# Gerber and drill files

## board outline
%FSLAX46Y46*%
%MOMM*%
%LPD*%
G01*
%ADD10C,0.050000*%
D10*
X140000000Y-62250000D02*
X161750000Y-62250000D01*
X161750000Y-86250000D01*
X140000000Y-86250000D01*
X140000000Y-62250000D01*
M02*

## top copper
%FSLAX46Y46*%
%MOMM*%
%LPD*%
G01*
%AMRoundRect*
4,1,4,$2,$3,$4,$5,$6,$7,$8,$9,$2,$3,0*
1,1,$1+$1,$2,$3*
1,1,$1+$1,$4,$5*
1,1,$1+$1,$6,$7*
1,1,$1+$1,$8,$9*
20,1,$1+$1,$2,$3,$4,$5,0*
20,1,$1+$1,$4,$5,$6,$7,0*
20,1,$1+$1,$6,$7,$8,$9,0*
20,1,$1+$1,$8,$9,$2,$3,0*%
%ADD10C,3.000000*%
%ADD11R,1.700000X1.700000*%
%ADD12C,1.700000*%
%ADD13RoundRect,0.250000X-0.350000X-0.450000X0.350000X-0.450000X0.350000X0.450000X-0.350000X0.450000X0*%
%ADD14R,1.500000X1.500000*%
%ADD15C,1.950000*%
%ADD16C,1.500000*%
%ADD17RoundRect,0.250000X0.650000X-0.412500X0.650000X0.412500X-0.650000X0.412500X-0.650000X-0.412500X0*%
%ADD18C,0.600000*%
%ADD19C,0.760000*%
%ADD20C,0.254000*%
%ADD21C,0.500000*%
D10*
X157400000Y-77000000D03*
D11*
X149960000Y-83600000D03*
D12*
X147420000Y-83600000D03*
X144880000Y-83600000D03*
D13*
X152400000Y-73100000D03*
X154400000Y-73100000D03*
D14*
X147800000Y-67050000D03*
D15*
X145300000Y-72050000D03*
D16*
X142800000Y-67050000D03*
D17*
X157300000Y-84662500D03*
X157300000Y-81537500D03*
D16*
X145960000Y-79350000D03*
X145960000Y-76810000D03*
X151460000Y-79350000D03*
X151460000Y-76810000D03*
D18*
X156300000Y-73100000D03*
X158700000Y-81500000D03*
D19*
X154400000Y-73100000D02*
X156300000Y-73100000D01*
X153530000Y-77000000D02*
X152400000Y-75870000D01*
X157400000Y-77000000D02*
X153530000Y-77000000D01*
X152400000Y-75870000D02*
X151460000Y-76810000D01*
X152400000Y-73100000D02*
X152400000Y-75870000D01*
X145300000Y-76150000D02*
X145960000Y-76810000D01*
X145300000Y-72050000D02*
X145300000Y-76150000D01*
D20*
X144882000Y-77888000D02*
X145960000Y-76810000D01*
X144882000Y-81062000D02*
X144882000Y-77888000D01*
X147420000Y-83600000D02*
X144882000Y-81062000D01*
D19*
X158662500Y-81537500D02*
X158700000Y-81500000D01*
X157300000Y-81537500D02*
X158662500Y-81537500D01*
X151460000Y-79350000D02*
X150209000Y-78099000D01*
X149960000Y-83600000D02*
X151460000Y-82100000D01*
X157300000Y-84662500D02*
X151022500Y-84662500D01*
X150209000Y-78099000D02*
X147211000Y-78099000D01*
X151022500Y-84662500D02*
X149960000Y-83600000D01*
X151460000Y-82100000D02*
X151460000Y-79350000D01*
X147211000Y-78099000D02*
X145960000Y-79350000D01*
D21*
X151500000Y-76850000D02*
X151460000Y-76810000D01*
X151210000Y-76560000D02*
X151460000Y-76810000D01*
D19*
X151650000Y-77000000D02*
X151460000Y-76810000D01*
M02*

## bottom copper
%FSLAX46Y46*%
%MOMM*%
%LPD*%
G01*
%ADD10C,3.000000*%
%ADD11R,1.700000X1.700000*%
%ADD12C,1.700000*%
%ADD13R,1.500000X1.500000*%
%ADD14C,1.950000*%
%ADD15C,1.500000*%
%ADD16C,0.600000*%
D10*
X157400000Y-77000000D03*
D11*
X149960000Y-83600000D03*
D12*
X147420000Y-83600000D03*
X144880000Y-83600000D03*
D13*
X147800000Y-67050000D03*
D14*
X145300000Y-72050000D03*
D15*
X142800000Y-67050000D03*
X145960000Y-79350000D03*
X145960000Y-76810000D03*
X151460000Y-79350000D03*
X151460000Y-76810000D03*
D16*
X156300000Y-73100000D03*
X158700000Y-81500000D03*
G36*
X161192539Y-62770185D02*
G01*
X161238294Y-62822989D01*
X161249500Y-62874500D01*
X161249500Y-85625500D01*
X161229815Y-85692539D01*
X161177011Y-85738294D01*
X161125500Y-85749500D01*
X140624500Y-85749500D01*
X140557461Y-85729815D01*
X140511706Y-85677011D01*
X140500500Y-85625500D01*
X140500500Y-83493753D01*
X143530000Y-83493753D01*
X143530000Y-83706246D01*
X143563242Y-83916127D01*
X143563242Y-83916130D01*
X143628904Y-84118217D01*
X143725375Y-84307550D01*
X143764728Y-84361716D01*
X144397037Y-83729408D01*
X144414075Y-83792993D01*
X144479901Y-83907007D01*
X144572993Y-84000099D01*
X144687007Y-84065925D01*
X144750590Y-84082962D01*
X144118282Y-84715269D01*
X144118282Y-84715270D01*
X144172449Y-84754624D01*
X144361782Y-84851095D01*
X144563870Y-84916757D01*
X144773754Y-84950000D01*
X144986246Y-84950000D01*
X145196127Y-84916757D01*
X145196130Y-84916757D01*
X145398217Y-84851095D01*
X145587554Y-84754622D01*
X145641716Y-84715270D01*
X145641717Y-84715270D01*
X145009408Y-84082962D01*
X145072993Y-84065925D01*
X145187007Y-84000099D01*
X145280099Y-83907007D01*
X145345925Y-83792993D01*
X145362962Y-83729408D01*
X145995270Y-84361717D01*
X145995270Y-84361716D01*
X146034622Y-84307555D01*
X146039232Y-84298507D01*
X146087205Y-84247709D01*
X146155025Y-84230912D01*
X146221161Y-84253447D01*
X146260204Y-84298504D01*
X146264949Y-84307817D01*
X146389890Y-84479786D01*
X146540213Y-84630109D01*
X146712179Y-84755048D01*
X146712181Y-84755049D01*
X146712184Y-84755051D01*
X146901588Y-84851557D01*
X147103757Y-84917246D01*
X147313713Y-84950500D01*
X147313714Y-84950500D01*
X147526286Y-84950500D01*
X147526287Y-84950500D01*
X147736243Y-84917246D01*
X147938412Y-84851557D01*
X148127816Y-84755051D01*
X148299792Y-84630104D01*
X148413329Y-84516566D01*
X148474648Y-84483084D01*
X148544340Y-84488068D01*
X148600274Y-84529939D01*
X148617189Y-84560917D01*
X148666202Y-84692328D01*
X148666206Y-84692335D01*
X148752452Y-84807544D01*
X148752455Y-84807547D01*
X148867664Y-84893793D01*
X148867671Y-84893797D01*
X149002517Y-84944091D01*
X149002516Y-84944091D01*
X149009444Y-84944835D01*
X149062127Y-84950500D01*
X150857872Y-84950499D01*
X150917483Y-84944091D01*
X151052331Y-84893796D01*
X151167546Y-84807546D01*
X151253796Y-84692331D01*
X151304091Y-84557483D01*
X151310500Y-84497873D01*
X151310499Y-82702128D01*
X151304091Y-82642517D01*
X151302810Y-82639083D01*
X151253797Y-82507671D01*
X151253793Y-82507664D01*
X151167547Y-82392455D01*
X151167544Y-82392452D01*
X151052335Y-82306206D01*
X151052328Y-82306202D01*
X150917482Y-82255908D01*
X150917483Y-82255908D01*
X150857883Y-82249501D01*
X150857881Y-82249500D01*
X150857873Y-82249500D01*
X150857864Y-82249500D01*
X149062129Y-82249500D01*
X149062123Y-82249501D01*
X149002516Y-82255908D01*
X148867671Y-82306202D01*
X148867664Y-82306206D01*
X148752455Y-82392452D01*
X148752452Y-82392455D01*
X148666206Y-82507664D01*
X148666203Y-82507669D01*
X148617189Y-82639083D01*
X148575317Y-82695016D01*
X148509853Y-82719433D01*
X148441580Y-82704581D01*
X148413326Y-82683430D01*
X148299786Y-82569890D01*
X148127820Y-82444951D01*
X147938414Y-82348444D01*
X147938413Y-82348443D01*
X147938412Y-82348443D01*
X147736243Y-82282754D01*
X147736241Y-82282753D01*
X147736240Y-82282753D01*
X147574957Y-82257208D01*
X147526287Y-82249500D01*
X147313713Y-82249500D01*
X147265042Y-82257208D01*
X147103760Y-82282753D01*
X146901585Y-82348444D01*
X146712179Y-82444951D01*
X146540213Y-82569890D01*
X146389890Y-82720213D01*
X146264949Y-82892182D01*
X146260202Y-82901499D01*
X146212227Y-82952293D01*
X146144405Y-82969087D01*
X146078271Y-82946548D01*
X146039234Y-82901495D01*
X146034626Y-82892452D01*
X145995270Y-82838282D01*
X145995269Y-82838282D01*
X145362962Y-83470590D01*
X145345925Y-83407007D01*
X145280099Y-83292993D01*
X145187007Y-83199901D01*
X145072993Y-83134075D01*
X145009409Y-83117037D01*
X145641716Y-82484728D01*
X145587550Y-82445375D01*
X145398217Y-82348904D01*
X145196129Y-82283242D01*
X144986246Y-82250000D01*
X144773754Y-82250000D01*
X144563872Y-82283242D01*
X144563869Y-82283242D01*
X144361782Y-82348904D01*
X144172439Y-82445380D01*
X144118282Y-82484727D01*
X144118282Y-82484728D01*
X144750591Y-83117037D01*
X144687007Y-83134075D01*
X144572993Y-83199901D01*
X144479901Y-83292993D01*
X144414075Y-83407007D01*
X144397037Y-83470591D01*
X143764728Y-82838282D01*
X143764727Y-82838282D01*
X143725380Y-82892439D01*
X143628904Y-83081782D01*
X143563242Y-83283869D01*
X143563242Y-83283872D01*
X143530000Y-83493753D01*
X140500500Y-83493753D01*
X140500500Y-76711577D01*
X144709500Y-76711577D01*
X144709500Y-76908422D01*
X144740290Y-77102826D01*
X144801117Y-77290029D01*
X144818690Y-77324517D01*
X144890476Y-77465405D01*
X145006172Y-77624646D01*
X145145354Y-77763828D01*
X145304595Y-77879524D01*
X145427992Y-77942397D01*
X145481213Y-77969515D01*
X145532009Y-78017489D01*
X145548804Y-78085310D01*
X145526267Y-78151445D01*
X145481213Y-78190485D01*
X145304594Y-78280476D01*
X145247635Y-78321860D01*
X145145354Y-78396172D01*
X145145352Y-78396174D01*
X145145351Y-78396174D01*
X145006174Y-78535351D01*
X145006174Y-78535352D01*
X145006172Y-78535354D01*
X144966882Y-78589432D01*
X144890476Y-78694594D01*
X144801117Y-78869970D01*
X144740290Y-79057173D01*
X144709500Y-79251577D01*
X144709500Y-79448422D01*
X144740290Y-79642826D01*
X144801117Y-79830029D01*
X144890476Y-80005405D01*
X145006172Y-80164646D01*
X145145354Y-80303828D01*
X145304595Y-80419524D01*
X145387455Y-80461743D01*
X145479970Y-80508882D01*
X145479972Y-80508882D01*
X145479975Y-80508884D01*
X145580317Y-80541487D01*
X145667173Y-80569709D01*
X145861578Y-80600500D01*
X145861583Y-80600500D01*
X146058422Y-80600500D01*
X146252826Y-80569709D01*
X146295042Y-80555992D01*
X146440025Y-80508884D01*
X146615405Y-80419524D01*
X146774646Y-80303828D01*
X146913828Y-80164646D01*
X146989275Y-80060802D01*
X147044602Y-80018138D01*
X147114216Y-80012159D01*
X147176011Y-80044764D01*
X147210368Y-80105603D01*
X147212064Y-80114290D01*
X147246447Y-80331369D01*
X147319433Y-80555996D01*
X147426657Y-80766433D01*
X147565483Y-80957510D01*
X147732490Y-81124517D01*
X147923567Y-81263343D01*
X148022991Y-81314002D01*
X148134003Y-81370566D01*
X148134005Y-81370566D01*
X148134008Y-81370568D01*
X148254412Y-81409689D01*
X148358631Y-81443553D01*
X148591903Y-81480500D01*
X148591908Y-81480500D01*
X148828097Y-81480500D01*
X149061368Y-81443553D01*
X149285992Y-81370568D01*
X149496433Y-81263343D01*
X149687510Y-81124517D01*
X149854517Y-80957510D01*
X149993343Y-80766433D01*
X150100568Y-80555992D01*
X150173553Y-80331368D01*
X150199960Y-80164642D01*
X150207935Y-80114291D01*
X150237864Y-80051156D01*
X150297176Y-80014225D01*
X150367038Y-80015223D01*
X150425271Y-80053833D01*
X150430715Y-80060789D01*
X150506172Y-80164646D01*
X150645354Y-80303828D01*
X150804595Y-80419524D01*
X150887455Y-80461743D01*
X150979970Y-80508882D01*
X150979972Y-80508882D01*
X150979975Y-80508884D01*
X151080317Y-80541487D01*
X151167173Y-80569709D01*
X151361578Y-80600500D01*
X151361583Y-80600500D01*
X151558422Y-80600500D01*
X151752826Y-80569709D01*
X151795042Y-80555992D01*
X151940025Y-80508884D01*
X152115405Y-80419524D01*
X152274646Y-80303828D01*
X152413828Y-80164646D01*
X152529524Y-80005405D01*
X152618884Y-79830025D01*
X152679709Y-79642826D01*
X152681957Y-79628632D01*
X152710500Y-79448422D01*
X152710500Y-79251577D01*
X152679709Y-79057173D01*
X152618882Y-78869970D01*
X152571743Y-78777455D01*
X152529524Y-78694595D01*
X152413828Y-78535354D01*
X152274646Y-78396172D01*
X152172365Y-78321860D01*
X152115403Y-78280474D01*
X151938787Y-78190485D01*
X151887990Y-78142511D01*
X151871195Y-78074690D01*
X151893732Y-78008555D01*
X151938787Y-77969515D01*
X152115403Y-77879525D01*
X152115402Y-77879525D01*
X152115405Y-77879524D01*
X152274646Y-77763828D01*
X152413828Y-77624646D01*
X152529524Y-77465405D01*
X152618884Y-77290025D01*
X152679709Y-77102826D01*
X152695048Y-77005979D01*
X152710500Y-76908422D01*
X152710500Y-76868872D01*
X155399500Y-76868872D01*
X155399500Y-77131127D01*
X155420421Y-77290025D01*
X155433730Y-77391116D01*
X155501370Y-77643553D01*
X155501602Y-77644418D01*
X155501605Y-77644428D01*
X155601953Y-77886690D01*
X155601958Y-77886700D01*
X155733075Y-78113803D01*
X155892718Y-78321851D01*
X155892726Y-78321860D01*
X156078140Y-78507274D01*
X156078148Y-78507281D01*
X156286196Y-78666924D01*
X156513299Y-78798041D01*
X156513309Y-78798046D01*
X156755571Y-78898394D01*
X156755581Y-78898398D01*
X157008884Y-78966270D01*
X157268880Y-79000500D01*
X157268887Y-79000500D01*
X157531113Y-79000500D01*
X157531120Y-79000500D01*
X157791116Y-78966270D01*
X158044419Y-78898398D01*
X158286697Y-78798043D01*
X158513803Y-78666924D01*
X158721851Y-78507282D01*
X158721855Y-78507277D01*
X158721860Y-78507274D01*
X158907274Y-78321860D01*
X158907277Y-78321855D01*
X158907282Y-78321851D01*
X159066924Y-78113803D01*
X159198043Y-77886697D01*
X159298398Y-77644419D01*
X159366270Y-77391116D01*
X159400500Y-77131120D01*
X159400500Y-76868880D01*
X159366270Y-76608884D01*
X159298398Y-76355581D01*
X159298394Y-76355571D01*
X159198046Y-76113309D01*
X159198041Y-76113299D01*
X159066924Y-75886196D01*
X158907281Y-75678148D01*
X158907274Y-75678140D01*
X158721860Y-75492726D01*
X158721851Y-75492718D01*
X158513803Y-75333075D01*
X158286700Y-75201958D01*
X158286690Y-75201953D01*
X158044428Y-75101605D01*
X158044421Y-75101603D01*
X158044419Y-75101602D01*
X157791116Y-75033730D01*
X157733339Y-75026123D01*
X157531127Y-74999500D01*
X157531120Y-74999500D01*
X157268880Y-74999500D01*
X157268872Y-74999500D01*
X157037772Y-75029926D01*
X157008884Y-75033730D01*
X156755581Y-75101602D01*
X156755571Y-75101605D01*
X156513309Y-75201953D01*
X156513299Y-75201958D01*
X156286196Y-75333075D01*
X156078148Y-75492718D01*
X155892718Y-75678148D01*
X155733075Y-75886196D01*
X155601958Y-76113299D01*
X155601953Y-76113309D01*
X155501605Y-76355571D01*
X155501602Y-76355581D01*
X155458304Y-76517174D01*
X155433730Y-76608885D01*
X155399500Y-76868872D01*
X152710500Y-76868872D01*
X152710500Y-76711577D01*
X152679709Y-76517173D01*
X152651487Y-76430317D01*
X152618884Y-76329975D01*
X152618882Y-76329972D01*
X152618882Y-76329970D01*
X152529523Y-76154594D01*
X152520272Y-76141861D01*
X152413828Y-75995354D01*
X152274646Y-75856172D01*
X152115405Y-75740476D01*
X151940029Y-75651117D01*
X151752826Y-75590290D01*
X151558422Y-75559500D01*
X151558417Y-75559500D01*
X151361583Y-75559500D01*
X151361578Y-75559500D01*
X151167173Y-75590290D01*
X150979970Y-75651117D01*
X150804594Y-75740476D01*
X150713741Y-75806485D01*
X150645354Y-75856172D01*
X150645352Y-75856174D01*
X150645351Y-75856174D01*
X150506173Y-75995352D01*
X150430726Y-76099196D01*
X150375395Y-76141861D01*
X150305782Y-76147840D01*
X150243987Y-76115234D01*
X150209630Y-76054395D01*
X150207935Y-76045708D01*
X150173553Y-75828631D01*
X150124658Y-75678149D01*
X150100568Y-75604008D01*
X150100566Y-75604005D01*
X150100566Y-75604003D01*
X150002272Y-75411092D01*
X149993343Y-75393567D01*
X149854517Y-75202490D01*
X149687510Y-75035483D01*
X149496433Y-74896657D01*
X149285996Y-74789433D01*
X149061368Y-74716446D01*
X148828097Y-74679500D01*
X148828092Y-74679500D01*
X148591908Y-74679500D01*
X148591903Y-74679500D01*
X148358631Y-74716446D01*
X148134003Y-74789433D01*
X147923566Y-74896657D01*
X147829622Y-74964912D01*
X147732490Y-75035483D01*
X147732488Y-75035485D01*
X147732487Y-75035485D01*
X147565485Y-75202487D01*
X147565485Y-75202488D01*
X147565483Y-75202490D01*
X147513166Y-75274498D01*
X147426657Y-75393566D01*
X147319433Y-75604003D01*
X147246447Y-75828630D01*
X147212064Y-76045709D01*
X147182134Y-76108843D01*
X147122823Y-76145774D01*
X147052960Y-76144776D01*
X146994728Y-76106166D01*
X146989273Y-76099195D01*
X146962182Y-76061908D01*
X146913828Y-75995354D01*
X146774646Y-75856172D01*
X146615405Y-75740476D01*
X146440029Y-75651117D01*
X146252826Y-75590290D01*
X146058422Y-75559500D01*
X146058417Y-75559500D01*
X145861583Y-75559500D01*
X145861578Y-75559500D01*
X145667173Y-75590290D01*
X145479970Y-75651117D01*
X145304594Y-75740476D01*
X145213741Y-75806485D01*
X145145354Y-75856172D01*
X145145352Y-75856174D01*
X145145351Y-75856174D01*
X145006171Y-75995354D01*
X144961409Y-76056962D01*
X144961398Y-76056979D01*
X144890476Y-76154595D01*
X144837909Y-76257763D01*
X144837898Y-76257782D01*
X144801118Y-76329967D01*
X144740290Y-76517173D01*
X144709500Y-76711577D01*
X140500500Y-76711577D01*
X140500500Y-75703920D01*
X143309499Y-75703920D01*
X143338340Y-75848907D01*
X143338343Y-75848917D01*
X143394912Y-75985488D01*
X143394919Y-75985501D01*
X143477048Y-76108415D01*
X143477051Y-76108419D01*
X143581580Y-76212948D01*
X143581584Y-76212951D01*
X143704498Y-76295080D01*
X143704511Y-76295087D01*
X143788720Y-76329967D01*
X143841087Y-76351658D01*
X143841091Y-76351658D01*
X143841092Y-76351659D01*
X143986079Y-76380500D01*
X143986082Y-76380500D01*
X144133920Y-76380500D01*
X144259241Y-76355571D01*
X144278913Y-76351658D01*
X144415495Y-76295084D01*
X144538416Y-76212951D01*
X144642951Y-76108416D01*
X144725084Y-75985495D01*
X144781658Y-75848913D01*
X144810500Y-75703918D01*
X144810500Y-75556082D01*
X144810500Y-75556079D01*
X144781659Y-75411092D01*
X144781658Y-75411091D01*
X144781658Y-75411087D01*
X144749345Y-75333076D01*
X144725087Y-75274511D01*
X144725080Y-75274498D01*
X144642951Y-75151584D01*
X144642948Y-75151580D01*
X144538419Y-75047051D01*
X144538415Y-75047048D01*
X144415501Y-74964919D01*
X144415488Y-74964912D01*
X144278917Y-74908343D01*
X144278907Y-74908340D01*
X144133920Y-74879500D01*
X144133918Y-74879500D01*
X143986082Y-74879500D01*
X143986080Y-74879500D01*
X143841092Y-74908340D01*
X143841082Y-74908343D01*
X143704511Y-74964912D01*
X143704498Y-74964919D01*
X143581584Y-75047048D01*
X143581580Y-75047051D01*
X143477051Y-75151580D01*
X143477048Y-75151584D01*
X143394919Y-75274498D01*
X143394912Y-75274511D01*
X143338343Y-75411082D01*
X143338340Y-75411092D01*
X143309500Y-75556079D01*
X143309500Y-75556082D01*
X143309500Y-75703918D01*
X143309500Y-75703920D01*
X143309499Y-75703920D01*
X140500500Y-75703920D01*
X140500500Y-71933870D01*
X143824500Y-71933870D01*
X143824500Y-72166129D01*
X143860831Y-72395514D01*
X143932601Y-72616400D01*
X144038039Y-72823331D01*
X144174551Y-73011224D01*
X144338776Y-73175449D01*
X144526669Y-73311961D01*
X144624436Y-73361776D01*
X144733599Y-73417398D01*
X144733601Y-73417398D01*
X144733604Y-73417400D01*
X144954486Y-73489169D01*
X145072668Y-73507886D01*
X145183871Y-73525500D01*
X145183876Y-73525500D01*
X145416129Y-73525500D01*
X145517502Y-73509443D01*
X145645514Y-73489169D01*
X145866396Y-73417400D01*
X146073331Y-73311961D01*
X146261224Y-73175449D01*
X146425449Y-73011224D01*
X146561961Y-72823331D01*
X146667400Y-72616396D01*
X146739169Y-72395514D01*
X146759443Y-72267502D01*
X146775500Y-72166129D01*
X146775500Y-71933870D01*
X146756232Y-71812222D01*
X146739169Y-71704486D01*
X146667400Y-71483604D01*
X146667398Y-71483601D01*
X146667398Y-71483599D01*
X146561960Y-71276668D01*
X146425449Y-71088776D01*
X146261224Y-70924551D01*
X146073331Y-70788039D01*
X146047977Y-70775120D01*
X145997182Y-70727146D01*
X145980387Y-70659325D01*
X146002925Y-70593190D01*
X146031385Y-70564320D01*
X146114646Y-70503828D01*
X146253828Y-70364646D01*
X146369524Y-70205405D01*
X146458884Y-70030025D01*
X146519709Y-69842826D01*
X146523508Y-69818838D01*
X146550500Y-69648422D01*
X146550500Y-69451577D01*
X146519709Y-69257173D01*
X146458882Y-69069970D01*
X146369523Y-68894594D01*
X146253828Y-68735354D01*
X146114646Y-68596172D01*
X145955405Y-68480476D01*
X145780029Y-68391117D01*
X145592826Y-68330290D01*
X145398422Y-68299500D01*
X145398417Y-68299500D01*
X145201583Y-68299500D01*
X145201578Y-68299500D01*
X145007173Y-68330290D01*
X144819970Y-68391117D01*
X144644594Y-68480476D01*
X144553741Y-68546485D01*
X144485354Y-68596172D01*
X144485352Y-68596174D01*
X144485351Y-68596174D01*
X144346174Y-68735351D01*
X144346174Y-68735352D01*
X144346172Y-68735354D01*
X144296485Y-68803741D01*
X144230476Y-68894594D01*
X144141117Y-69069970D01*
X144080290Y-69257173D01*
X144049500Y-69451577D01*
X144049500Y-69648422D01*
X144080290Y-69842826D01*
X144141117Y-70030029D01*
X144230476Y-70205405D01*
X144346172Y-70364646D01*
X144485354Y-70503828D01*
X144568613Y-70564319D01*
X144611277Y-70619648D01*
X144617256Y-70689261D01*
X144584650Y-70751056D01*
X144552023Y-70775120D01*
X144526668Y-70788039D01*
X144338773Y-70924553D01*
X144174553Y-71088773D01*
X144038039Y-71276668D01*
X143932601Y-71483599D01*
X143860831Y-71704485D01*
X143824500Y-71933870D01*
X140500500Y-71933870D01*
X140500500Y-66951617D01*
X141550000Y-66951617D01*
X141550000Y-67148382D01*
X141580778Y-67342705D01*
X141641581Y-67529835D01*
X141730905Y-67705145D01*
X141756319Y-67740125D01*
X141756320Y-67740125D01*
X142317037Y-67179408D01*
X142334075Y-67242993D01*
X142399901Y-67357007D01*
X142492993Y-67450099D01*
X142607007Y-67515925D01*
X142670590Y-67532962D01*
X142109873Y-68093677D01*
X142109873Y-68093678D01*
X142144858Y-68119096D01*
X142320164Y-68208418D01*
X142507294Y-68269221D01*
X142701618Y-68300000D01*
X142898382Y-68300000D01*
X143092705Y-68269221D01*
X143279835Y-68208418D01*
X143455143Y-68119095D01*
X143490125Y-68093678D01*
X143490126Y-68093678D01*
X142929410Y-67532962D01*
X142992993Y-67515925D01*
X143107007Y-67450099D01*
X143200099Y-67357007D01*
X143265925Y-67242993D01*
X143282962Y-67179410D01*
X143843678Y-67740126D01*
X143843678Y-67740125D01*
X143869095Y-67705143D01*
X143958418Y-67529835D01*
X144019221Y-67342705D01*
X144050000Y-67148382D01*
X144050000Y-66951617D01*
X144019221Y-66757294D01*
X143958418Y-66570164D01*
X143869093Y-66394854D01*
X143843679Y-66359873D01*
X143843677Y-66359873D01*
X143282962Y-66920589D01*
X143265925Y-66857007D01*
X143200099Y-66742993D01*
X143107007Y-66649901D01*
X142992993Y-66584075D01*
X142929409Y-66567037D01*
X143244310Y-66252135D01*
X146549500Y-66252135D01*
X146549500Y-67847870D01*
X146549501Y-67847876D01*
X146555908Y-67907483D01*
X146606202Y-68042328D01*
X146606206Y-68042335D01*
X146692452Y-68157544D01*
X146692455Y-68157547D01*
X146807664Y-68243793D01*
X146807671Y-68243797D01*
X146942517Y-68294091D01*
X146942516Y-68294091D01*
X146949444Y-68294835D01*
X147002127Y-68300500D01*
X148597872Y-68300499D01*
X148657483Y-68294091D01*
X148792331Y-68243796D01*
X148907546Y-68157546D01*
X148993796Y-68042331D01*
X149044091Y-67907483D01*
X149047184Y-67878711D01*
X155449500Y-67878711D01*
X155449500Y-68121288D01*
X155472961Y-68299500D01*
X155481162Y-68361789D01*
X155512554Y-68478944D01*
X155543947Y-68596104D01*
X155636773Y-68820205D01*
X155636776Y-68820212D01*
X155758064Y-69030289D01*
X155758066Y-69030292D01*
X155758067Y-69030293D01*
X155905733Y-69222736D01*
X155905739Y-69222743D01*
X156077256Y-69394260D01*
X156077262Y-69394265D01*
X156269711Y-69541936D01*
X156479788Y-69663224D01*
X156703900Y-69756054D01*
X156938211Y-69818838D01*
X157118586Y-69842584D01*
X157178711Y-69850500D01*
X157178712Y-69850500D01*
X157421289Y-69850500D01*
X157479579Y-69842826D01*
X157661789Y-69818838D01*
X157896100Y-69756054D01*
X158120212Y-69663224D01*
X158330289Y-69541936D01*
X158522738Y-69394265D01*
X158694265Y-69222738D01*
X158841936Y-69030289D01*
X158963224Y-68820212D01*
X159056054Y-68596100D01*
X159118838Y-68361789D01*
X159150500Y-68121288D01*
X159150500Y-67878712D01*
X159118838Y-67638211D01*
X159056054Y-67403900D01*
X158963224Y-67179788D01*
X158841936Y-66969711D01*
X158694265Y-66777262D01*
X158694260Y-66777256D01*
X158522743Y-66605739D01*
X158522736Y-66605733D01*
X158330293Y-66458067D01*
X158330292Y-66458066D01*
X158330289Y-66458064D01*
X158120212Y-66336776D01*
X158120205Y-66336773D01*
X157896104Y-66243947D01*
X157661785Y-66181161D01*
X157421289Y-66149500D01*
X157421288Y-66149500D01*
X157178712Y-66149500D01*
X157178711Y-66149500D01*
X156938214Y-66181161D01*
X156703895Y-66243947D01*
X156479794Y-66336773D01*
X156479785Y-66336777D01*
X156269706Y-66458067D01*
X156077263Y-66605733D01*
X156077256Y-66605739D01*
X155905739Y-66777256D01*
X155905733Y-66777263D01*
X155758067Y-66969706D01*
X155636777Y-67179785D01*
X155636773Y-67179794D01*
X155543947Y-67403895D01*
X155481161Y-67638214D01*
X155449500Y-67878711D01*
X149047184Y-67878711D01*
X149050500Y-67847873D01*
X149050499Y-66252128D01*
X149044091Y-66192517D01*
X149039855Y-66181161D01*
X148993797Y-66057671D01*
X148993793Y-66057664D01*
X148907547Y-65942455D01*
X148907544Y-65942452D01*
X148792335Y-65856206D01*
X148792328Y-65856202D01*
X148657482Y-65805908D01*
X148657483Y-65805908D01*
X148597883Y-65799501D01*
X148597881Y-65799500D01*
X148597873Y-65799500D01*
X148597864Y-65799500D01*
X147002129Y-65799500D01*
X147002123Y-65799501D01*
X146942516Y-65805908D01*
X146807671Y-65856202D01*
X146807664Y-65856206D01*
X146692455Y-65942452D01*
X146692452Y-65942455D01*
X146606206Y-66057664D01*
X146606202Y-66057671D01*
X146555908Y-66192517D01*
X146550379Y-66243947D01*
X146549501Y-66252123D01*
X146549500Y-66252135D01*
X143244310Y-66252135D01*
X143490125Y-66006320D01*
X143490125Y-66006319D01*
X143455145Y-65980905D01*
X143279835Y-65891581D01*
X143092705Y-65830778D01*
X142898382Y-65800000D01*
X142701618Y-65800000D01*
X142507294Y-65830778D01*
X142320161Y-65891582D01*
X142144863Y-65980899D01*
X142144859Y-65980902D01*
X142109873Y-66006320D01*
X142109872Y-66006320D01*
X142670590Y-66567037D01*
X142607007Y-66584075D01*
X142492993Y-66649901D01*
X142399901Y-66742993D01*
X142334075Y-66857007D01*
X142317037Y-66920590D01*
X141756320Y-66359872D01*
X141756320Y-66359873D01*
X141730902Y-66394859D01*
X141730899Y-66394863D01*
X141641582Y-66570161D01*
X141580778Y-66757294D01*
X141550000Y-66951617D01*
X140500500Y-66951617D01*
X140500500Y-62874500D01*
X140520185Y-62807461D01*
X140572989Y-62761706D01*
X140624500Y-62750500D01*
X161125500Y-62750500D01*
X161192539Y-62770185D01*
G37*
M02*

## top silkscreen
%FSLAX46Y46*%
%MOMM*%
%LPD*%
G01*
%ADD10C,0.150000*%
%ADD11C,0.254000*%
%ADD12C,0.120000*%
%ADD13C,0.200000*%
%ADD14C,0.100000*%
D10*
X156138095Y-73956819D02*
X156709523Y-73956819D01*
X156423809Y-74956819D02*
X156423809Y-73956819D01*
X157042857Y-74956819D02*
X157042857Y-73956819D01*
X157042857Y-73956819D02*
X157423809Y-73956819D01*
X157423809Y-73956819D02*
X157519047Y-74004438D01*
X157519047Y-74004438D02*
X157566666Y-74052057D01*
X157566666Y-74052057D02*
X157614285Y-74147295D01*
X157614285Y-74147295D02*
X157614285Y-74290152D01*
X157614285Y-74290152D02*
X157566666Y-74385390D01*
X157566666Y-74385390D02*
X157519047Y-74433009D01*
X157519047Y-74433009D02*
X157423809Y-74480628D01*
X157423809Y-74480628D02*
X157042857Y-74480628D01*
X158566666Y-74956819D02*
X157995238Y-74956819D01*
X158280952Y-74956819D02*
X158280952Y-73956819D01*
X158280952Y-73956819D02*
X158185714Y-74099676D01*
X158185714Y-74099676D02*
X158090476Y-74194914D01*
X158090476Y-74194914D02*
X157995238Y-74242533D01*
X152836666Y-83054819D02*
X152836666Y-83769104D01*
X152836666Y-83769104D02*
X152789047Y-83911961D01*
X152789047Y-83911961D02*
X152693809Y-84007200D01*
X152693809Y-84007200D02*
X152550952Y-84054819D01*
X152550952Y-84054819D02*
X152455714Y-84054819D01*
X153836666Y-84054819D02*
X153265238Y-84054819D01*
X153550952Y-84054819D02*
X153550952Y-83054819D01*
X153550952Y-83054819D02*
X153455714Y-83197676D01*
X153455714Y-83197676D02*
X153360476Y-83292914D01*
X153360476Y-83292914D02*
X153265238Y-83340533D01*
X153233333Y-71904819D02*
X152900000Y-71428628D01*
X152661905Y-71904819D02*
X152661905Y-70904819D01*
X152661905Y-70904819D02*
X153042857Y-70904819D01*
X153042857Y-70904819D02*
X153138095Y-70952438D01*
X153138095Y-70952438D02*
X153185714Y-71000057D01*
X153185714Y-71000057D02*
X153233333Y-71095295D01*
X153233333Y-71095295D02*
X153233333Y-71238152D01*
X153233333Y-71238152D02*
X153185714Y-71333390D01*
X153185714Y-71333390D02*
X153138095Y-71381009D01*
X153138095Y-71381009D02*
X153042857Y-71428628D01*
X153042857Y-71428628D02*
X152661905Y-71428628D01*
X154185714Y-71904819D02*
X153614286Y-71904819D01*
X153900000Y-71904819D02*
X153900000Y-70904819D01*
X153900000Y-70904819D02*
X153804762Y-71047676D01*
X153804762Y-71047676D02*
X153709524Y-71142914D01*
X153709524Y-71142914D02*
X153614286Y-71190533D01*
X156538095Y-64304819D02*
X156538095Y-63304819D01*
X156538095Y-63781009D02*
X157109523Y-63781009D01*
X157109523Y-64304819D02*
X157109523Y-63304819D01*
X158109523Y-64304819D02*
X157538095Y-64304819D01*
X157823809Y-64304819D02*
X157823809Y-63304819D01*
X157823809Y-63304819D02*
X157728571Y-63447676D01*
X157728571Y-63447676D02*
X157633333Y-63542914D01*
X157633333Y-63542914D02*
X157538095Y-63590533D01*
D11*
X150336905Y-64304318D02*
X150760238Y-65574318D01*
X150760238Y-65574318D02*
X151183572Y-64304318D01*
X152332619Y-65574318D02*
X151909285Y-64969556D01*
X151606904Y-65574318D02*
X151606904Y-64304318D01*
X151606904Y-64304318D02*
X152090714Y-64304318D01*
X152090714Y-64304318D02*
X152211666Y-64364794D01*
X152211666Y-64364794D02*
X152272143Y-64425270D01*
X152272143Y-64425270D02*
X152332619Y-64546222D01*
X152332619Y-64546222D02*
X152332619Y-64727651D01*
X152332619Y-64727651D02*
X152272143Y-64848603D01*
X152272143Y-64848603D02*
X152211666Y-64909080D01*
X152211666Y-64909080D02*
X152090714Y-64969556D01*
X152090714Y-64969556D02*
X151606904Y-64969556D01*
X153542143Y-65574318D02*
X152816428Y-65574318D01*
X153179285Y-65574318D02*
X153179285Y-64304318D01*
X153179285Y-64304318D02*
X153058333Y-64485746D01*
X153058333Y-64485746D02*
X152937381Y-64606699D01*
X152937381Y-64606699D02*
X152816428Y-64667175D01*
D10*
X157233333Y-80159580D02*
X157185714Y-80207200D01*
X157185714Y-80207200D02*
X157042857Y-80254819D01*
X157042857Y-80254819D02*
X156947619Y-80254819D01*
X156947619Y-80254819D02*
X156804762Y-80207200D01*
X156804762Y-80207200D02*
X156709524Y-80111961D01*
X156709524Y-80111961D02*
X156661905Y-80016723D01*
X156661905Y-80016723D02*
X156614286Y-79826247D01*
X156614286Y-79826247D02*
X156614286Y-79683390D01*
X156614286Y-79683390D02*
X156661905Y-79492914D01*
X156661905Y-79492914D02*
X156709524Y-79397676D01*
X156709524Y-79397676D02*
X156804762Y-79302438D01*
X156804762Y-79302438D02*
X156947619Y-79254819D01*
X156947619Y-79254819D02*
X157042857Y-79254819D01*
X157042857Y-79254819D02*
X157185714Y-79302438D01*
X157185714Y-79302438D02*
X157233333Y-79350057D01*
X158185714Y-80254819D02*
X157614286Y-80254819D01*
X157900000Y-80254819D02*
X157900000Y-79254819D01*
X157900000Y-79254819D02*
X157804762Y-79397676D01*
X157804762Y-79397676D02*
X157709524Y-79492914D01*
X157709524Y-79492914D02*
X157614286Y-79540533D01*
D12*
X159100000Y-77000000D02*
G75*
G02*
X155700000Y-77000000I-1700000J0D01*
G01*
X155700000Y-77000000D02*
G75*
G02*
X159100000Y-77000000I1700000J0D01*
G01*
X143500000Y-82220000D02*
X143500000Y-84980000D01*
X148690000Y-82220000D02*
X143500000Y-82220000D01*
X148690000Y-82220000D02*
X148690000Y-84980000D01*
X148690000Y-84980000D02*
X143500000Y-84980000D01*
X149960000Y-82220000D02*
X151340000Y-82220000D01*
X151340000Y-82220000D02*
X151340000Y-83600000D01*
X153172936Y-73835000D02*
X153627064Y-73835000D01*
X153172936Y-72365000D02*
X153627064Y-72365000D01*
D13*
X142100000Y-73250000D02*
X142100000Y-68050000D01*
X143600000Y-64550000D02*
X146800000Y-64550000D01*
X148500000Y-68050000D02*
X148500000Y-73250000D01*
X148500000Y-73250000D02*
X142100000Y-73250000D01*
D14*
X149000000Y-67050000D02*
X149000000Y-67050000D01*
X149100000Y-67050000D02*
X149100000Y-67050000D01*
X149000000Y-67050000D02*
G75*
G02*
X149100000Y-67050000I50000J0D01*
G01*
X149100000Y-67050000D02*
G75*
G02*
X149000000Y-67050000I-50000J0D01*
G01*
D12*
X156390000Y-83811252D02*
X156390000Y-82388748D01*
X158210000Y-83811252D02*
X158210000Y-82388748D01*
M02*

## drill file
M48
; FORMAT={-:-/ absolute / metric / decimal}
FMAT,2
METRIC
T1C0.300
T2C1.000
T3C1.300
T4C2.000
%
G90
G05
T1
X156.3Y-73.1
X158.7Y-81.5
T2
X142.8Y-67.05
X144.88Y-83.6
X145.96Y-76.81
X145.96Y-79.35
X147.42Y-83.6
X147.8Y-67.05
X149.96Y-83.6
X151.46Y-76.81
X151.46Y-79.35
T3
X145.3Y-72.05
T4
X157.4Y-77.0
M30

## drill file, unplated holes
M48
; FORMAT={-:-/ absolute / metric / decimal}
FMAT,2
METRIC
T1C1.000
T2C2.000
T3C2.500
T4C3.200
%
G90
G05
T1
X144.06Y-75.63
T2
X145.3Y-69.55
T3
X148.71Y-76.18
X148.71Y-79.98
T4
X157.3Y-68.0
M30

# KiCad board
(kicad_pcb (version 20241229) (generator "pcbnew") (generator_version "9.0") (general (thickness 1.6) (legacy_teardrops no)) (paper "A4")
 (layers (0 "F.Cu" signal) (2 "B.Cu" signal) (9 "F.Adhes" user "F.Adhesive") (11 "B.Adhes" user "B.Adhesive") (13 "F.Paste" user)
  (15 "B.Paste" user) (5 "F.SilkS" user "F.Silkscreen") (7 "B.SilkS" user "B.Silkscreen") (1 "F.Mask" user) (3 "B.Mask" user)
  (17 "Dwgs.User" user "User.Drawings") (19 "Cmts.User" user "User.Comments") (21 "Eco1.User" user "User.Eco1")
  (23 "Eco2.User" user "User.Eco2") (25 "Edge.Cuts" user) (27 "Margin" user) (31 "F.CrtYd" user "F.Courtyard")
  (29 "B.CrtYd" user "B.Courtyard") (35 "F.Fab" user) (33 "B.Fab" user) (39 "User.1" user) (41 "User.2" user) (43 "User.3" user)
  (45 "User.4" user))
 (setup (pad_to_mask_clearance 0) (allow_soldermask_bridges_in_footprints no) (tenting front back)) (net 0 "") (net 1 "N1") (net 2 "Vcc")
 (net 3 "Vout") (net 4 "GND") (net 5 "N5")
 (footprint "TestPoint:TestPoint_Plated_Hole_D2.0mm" (layer "F.Cu") (at 157.4 77)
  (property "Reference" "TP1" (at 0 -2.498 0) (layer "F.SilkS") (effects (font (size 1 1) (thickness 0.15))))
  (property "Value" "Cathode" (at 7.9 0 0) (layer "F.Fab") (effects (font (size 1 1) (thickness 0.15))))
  (fp_circle (center 0 0) (end 0 -1.7) (stroke (width 0.12) (type solid)) (fill no) (layer "F.SilkS"))
  (pad "1" thru_hole circle (at 0 0) (size 3 3) (drill 2) (layers "*.Cu" "*.Mask") (remove_unused_layers no) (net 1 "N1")))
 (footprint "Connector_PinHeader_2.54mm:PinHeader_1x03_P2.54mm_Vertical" (layer "F.Cu") (at 149.96 83.6 -90)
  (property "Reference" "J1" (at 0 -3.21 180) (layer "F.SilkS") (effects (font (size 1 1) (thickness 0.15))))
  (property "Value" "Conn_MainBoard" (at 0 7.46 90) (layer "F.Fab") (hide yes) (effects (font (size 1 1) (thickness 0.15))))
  (fp_line (start -1.38 6.46) (end 1.38 6.46) (stroke (width 0.12) (type solid)) (layer "F.SilkS"))
  (fp_line (start -1.38 1.27) (end -1.38 6.46) (stroke (width 0.12) (type solid)) (layer "F.SilkS"))
  (fp_line (start -1.38 1.27) (end 1.38 1.27) (stroke (width 0.12) (type solid)) (layer "F.SilkS"))
  (fp_line (start 1.38 1.27) (end 1.38 6.46) (stroke (width 0.12) (type solid)) (layer "F.SilkS"))
  (fp_line (start -1.38 0) (end -1.38 -1.38) (stroke (width 0.12) (type solid)) (layer "F.SilkS"))
  (fp_line (start -1.38 -1.38) (end 0 -1.38) (stroke (width 0.12) (type solid)) (layer "F.SilkS"))
  (pad "1" thru_hole rect (at 0 0 270) (size 1.7 1.7) (drill 1) (layers "*.Cu" "*.Mask") (remove_unused_layers no) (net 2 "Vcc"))
  (pad "2" thru_hole circle (at 0 2.54 270) (size 1.7 1.7) (drill 1) (layers "*.Cu" "*.Mask") (remove_unused_layers no) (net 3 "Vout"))
  (pad "3" thru_hole circle (at 0 5.08 270) (size 1.7 1.7) (drill 1) (layers "*.Cu" "*.Mask") (remove_unused_layers no) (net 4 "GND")))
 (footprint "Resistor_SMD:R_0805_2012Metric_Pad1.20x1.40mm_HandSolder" (layer "F.Cu") (at 153.4 73.1)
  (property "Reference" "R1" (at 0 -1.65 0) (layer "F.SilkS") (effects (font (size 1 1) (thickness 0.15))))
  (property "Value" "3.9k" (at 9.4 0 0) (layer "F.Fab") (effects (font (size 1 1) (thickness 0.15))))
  (fp_line (start -0.227064 -0.735) (end 0.227064 -0.735) (stroke (width 0.12) (type solid)) (layer "F.SilkS"))
  (fp_line (start -0.227064 0.735) (end 0.227064 0.735) (stroke (width 0.12) (type solid)) (layer "F.SilkS"))
  (pad "1" smd roundrect (at -1 0) (size 1.2 1.4) (layers "F.Cu" "F.Mask" "F.Paste") (roundrect_rratio 0.208333) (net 1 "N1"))
  (pad "2" smd roundrect (at 1 0) (size 1.2 1.4) (layers "F.Cu" "F.Mask" "F.Paste") (roundrect_rratio 0.208333) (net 4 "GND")))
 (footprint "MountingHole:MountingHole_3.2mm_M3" (layer "F.Cu") (at 157.3 68)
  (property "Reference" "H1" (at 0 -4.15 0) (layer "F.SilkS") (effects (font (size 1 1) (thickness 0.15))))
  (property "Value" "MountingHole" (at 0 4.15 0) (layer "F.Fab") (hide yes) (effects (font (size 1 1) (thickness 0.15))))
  (pad "" np_thru_hole circle (at 0 0) (size 3.2 3.2) (drill 3.2) (layers "*.Cu" "*.Mask")))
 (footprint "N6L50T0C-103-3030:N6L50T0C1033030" (layer "F.Cu") (at 147.8 67.05 180)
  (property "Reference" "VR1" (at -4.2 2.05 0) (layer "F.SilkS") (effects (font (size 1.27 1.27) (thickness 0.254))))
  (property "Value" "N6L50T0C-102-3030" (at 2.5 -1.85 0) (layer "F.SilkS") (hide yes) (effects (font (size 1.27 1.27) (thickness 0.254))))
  (fp_line (start 5.7 -6.2) (end 5.7 -1) (stroke (width 0.2) (type solid)) (layer "F.SilkS"))
  (fp_line (start 4.2 2.5) (end 1 2.5) (stroke (width 0.2) (type solid)) (layer "F.SilkS"))
  (fp_line (start -0.7 -1) (end -0.7 -6.2) (stroke (width 0.2) (type solid)) (layer "F.SilkS"))
  (fp_line (start -0.7 -6.2) (end 5.7 -6.2) (stroke (width 0.2) (type solid)) (layer "F.SilkS"))
  (fp_line (start -1.2 0) (end -1.2 0) (stroke (width 0.1) (type solid)) (layer "F.SilkS"))
  (fp_line (start -1.3 0) (end -1.3 0) (stroke (width 0.1) (type solid)) (layer "F.SilkS"))
  (fp_arc (start -1.2 0) (mid -1.25 0.05) (end -1.3 0) (stroke (width 0.1) (type solid)) (layer "F.SilkS"))
  (fp_arc (start -1.3 0) (mid -1.25 -0.05) (end -1.2 0) (stroke (width 0.1) (type solid)) (layer "F.SilkS"))
  (pad "" np_thru_hole circle (at 2.5 -2.5 180) (size 2 2) (drill 2) (layers "*.Cu" "*.Mask"))
  (pad "1" thru_hole rect (at 0 0 180) (size 1.5 1.5) (drill 1) (layers "*.Cu" "*.Mask") (remove_unused_layers no) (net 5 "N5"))
  (pad "2" thru_hole circle (at 2.5 -5 180) (size 1.95 1.95) (drill 1.3) (layers "*.Cu" "*.Mask") (remove_unused_layers no) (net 3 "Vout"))
  (pad "3" thru_hole circle (at 5 0 180) (size 1.5 1.5) (drill 1) (layers "*.Cu" "*.Mask") (remove_unused_layers no) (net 4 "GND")))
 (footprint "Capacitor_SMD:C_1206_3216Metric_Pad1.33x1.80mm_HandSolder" (layer "F.Cu") (at 157.3 83.1 90)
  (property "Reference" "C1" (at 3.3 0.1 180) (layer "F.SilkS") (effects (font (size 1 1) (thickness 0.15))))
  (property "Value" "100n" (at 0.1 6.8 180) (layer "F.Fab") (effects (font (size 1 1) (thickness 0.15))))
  (fp_line (start -0.711252 -0.91) (end 0.711252 -0.91) (stroke (width 0.12) (type solid)) (layer "F.SilkS"))
  (fp_line (start -0.711252 0.91) (end 0.711252 0.91) (stroke (width 0.12) (type solid)) (layer "F.SilkS"))
  (pad "1" smd roundrect (at -1.5625 0 90) (size 1.325 1.8) (layers "F.Cu" "F.Mask" "F.Paste") (roundrect_rratio 0.188679) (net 2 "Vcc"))
  (pad "2" smd roundrect (at 1.5625 0 90) (size 1.325 1.8) (layers "F.Cu" "F.Mask" "F.Paste") (roundrect_rratio 0.188679) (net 4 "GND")))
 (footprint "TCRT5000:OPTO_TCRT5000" (layer "B.Cu") (at 148.71 78.08)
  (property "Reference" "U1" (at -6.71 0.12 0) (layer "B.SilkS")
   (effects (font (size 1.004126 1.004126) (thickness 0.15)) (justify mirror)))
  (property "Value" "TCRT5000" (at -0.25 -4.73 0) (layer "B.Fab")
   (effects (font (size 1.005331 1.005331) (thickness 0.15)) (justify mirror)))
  (pad "" np_thru_hole circle (at -4.65 -2.45) (size 1 1) (drill 1) (layers "*.Cu" "*.Mask"))
  (pad "" np_thru_hole circle (at 0 -1.9) (size 2.5 2.5) (drill 2.5) (layers "*.Cu" "*.Mask"))
  (pad "" np_thru_hole circle (at 0 1.9) (size 2.5 2.5) (drill 2.5) (layers "*.Cu" "*.Mask"))
  (pad "1" thru_hole circle (at -2.75 1.27) (size 1.5 1.5) (drill 1) (layers "*.Cu" "*.Mask") (remove_unused_layers no) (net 2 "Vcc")
   (solder_mask_margin 0.102))
  (pad "2" thru_hole circle (at -2.75 -1.27) (size 1.5 1.5) (drill 1) (layers "*.Cu" "*.Mask") (remove_unused_layers no) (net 3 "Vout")
   (solder_mask_margin 0.102))
  (pad "3" thru_hole circle (at 2.75 1.27) (size 1.5 1.5) (drill 1) (layers "*.Cu" "*.Mask") (remove_unused_layers no) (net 2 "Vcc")
   (solder_mask_margin 0.102))
  (pad "4" thru_hole circle (at 2.75 -1.27) (size 1.5 1.5) (drill 1) (layers "*.Cu" "*.Mask") (remove_unused_layers no) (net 1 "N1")
   (solder_mask_margin 0.102)))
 (gr_rect (start 140 62.25) (end 161.75 86.25) (stroke (width 0.05) (type default)) (fill no) (locked yes) (layer "Edge.Cuts"))
 (segment (start 144.882 77.888) (end 145.96 76.81) (width 0.254) (layer "F.Cu") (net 3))
 (segment (start 145.3 72.05) (end 145.3 76.15) (width 0.76) (layer "F.Cu") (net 3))
 (segment (start 145.3 76.15) (end 145.96 76.81) (width 0.76) (layer "F.Cu") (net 3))
 (segment (start 144.882 81.062) (end 144.882 77.888) (width 0.254) (layer "F.Cu") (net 3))
 (segment (start 147.42 83.6) (end 144.882 81.062) (width 0.254) (layer "F.Cu") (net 3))
 (segment (start 154.4 73.1) (end 156.3 73.1) (width 0.76) (layer "F.Cu") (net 4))
 (segment (start 158.6625 81.5375) (end 158.7 81.5) (width 0.76) (layer "F.Cu") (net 4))
 (segment (start 157.3 81.5375) (end 158.6625 81.5375) (width 0.76) (layer "F.Cu") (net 4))
 (via (at 156.3 73.1) (size 0.6) (drill 0.3) (layers "F.Cu" "B.Cu") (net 4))
 (via (at 158.7 81.5) (size 0.6) (drill 0.3) (layers "F.Cu" "B.Cu") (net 4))
 (segment (start 151.46 79.35) (end 150.209 78.099) (width 0.76) (layer "F.Cu") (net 2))
 (segment (start 149.96 83.6) (end 151.46 82.1) (width 0.76) (layer "F.Cu") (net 2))
 (segment (start 157.3 84.6625) (end 151.0225 84.6625) (width 0.76) (layer "F.Cu") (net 2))
 (segment (start 150.209 78.099) (end 147.211 78.099) (width 0.76) (layer "F.Cu") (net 2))
 (segment (start 151.0225 84.6625) (end 149.96 83.6) (width 0.76) (layer "F.Cu") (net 2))
 (segment (start 151.46 82.1) (end 151.46 79.35) (width 0.76) (layer "F.Cu") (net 2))
 (segment (start 147.211 78.099) (end 145.96 79.35) (width 0.76) (layer "F.Cu") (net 2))
 (segment (start 151.5 76.85) (end 151.46 76.81) (width 0.5) (layer "F.Cu") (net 1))
 (segment (start 152.4 73.1) (end 152.4 75.87) (width 0.76) (layer "F.Cu") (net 1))
 (segment (start 151.21 76.56) (end 151.46 76.81) (width 0.5) (layer "F.Cu") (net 1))
 (segment (start 152.4 75.87) (end 151.46 76.81) (width 0.76) (layer "F.Cu") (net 1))
 (segment (start 151.65 77) (end 151.46 76.81) (width 0.76) (layer "F.Cu") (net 1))
 (segment (start 157.4 77) (end 153.53 77) (width 0.76) (layer "F.Cu") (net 1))
 (segment (start 153.53 77) (end 152.4 75.87) (width 0.76) (layer "F.Cu") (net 1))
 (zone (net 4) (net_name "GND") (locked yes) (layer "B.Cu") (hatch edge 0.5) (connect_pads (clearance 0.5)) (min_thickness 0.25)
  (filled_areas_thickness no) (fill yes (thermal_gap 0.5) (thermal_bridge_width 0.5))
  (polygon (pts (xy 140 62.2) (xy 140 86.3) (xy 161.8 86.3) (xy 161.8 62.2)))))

